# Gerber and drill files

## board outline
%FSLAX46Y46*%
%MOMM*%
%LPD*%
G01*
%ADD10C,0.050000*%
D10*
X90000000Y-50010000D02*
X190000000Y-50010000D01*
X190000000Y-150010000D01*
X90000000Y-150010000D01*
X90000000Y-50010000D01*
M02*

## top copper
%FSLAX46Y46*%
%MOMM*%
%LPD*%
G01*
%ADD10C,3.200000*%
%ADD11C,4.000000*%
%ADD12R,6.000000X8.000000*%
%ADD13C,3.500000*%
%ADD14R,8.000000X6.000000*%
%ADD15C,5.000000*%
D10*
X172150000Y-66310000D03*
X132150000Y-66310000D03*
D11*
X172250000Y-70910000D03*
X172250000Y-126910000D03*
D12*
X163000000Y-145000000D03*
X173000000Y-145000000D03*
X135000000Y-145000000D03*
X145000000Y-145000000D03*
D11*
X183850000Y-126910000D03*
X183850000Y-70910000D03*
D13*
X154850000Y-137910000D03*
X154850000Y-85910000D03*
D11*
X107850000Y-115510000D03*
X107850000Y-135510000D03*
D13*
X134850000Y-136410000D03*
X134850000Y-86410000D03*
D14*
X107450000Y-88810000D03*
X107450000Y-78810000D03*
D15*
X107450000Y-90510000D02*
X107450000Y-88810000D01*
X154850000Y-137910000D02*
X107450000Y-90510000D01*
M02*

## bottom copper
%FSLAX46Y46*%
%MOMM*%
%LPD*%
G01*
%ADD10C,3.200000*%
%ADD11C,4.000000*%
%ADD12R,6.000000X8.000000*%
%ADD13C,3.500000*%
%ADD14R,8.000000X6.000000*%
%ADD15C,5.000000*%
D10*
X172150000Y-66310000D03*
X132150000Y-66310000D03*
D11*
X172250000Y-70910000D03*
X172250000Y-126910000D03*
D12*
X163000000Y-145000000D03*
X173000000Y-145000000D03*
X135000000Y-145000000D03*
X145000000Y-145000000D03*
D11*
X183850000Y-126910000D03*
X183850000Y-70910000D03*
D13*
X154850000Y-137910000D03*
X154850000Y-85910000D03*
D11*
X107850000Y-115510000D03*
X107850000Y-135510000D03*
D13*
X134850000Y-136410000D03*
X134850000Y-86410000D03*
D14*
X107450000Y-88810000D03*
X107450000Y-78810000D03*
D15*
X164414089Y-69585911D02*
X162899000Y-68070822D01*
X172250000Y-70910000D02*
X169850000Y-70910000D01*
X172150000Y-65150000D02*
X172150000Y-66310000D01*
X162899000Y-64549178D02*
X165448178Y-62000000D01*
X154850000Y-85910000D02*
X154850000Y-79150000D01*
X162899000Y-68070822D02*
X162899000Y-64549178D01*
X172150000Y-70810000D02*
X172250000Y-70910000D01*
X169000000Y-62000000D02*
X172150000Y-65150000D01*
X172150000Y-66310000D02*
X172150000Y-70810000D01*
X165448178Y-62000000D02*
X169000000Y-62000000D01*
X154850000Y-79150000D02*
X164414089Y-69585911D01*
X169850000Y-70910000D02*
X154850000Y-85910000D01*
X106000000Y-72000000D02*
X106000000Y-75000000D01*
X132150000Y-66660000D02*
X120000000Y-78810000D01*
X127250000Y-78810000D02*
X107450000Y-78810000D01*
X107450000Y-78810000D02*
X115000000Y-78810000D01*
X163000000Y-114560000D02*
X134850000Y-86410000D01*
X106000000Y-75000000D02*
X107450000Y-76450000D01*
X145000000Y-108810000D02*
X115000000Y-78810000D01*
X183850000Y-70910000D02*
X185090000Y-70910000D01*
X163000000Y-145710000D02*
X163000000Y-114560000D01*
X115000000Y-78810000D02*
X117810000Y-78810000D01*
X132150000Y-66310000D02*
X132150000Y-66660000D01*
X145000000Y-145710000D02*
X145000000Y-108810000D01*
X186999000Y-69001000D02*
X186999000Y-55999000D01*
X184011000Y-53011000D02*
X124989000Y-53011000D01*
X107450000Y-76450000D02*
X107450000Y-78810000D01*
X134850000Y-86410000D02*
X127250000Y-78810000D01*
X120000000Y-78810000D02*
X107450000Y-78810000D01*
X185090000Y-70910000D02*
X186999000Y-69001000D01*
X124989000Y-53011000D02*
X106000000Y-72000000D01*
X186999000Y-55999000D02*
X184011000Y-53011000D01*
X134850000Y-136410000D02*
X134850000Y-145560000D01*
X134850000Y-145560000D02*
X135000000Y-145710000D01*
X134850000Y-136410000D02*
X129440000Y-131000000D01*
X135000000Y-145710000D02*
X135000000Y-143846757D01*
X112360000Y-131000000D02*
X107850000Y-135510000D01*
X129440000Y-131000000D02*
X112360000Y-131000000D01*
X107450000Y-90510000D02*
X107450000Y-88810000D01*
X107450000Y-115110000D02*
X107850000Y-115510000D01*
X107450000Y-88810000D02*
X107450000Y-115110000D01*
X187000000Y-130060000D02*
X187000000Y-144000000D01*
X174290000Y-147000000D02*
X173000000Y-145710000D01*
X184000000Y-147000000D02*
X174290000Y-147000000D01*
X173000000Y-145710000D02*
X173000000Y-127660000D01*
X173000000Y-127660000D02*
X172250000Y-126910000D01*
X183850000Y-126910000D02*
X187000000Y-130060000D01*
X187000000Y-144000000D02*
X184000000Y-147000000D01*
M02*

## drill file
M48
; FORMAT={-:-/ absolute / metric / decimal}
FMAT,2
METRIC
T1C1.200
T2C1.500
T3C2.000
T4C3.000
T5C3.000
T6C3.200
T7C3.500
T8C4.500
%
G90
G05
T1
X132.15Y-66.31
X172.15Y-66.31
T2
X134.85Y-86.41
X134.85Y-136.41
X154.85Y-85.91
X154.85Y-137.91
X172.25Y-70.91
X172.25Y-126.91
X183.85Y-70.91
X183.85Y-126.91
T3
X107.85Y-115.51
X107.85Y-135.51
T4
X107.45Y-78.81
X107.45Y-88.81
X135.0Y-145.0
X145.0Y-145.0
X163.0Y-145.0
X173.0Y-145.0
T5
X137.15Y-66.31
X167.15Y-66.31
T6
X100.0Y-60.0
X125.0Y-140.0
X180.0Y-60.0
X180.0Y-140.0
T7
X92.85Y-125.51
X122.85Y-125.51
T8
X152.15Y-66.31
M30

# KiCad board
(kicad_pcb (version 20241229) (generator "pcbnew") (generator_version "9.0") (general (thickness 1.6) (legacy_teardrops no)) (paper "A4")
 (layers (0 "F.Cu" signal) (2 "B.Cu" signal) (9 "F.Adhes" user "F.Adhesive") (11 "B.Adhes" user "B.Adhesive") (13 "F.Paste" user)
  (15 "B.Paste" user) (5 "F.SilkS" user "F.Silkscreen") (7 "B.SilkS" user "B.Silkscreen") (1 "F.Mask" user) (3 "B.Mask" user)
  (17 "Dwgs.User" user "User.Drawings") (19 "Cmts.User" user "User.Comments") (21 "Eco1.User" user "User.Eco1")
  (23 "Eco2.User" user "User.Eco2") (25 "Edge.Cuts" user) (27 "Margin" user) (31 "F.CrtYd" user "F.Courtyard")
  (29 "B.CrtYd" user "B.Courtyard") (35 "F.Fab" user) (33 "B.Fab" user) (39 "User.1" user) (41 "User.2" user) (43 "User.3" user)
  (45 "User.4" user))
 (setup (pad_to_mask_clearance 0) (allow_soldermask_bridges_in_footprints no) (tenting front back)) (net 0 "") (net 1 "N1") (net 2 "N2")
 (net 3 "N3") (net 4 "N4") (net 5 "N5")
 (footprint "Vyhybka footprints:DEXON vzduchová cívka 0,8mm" (layer "F.Cu") (at 152.15 66.31 180)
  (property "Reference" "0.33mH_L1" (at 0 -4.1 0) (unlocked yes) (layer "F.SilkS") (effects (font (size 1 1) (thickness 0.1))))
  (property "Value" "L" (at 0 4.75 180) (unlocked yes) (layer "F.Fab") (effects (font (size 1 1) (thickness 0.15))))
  (pad "" np_thru_hole circle (at -15 0 180) (size 3 3) (drill 3) (layers "*.Cu" "*.Mask"))
  (pad "" np_thru_hole circle (at 0 0 180) (size 4.5 4.5) (drill 4.5) (layers "*.Cu" "*.Mask"))
  (pad "" np_thru_hole circle (at 15 0 180) (size 3 3) (drill 3) (layers "*.Cu" "*.Mask"))
  (pad "1" thru_hole circle (at -20 0 180) (size 3.2 3.2) (drill 1.2) (layers "*.Cu" "*.Mask") (remove_unused_layers no) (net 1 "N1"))
  (pad "2" thru_hole circle (at 20 0 180) (size 3.2 3.2) (drill 1.2) (layers "*.Cu" "*.Mask") (remove_unused_layers no) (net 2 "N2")))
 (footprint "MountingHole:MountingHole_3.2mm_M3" (layer "F.Cu") (at 180 60)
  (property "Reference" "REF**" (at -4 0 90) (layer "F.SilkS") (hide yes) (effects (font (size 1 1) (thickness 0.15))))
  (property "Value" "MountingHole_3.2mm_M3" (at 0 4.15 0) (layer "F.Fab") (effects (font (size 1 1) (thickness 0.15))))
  (pad "" np_thru_hole circle (at 0 0) (size 3.2 3.2) (drill 3.2) (layers "*.Cu" "*.Mask")))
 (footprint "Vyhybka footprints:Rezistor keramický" (layer "F.Cu") (at 172.25 98.91 -90)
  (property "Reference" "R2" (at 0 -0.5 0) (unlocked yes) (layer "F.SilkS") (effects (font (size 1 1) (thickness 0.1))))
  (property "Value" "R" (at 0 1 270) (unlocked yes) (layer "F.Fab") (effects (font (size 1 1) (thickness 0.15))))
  (pad "1" thru_hole circle (at -28 0 270) (size 4 4) (drill 1.5) (layers "*.Cu" "*.Mask") (remove_unused_layers no) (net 1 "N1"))
  (pad "2" thru_hole circle (at 28 0 270) (size 4 4) (drill 1.5) (layers "*.Cu" "*.Mask") (remove_unused_layers no) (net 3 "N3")))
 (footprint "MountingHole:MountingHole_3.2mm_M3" (layer "F.Cu") (at 100 60)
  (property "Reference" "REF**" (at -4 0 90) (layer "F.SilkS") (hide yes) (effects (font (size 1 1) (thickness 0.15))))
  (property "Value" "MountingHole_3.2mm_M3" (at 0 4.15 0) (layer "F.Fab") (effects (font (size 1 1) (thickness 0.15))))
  (pad "" np_thru_hole circle (at 0 0) (size 3.2 3.2) (drill 3.2) (layers "*.Cu" "*.Mask")))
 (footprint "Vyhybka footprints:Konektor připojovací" (layer "F.Cu") (at 168 145)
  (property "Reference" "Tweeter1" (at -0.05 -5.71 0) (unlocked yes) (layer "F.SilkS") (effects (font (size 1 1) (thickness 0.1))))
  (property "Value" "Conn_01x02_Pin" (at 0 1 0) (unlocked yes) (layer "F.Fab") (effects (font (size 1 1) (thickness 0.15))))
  (pad "1" thru_hole rect (at -5 0) (size 6 8) (drill 3) (layers "*.Cu" "*.Mask") (remove_unused_layers no) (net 2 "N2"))
  (pad "2" thru_hole rect (at 5 0) (size 6 8) (drill 3) (layers "*.Cu" "*.Mask") (remove_unused_layers no) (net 3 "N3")))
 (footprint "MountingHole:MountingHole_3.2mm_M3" (layer "F.Cu") (at 125 140)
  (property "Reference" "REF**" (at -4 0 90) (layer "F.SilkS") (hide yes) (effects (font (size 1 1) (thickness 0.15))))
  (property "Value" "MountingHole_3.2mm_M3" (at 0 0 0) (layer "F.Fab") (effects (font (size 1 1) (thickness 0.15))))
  (pad "" np_thru_hole circle (at 0 0) (size 3.2 3.2) (drill 3.2) (layers "*.Cu" "*.Mask")))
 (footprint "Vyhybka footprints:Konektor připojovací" (layer "F.Cu") (at 140 145)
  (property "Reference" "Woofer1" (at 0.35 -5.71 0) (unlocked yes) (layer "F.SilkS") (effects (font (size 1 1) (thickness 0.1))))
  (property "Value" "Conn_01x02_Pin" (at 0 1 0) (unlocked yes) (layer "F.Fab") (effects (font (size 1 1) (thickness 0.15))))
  (pad "1" thru_hole rect (at -5 0) (size 6 8) (drill 3) (layers "*.Cu" "*.Mask") (remove_unused_layers no) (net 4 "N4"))
  (pad "2" thru_hole rect (at 5 0) (size 6 8) (drill 3) (layers "*.Cu" "*.Mask") (remove_unused_layers no) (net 2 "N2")))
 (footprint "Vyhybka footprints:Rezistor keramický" (layer "F.Cu") (at 183.85 98.91 90)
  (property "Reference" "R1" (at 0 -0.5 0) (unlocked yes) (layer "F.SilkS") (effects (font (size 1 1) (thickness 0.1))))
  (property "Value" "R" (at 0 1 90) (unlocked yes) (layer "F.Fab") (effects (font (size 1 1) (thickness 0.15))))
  (pad "1" thru_hole circle (at -28 0 90) (size 4 4) (drill 1.5) (layers "*.Cu" "*.Mask") (remove_unused_layers no) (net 3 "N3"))
  (pad "2" thru_hole circle (at 28 0 90) (size 4 4) (drill 1.5) (layers "*.Cu" "*.Mask") (remove_unused_layers no) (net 2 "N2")))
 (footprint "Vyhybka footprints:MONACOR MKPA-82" (layer "F.Cu") (at 154.85 111.91 90)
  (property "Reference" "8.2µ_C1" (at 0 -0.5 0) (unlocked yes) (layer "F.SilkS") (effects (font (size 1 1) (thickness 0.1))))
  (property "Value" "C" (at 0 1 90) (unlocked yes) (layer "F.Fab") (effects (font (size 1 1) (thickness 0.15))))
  (pad "1" thru_hole circle (at -26 0 90) (size 3.5 3.5) (drill 1.5) (layers "*.Cu" "*.Mask") (remove_unused_layers no) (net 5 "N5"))
  (pad "2" thru_hole circle (at 26 0 90) (size 3.5 3.5) (drill 1.5) (layers "*.Cu" "*.Mask") (remove_unused_layers no) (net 1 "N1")))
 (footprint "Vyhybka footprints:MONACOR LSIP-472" (layer "F.Cu") (at 107.85 125.51 -90)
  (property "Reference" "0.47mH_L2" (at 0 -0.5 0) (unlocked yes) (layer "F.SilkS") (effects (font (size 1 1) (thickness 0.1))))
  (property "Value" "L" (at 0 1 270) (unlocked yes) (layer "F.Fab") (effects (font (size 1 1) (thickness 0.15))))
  (pad "" np_thru_hole circle (at 0 -15 270) (size 3.5 3.5) (drill 3.5) (layers "*.Cu" "*.Mask"))
  (pad "" np_thru_hole circle (at 0 15 270) (size 3.5 3.5) (drill 3.5) (layers "*.Cu" "*.Mask"))
  (pad "1" thru_hole circle (at -10 0 270) (size 4 4) (drill 2) (layers "*.Cu" "*.Mask") (remove_unused_layers no) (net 5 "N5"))
  (pad "2" thru_hole circle (at 10 0 270) (size 4 4) (drill 2) (layers "*.Cu" "*.Mask") (remove_unused_layers no) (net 4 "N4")))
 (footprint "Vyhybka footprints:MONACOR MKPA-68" (layer "F.Cu") (at 134.85 111.41 90)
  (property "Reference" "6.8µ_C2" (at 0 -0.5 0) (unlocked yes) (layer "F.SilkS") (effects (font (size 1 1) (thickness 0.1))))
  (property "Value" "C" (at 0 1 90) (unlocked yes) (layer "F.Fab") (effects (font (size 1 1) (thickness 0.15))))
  (pad "1" thru_hole circle (at -25 0 90) (size 3.5 3.5) (drill 1.5) (layers "*.Cu" "*.Mask") (remove_unused_layers no) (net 4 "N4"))
  (pad "2" thru_hole circle (at 25 0 90) (size 3.5 3.5) (drill 1.5) (layers "*.Cu" "*.Mask") (remove_unused_layers no) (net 2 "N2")))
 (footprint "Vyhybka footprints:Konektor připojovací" (layer "F.Cu") (at 107.45 83.81 90)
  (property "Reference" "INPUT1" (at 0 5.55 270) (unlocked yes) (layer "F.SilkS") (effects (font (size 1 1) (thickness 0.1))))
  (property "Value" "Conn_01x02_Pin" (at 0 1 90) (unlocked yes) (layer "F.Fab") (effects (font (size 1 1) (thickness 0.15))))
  (pad "1" thru_hole rect (at -5 0 90) (size 6 8) (drill 3) (layers "*.Cu" "*.Mask") (remove_unused_layers no) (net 5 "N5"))
  (pad "2" thru_hole rect (at 5 0 90) (size 6 8) (drill 3) (layers "*.Cu" "*.Mask") (remove_unused_layers no) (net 2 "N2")))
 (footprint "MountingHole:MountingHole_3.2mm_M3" (layer "F.Cu") (at 180 140)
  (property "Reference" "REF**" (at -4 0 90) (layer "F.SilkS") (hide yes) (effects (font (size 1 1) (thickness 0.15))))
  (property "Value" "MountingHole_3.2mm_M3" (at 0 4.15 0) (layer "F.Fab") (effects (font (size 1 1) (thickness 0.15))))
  (pad "" np_thru_hole circle (at 0 0) (size 3.2 3.2) (drill 3.2) (layers "*.Cu" "*.Mask")))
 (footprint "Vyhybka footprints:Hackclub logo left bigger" (layer "F.Cu") (at 102 69)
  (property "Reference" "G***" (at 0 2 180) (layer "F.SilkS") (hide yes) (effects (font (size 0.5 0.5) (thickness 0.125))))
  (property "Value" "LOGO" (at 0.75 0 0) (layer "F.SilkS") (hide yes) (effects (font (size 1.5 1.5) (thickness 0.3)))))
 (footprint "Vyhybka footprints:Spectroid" (layer "B.Cu") (at 98 137 180)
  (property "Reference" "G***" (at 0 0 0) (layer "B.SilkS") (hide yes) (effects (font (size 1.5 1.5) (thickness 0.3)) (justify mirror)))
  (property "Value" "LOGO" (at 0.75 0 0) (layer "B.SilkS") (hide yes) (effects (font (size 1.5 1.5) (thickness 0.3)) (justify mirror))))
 (gr_rect (start 90 50.01) (end 190 150.01) (stroke (width 0.05) (type default)) (fill no) (layer "Edge.Cuts"))
 (segment (start 164.414089 69.585911) (end 162.899 68.070822) (width 5) (layer "B.Cu") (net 1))
 (segment (start 172.25 70.91) (end 169.85 70.91) (width 5) (layer "B.Cu") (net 1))
 (segment (start 172.15 65.15) (end 172.15 66.31) (width 5) (layer "B.Cu") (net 1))
 (segment (start 162.899 64.549178) (end 165.448178 62) (width 5) (layer "B.Cu") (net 1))
 (segment (start 154.85 85.91) (end 154.85 79.15) (width 5) (layer "B.Cu") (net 1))
 (segment (start 162.899 68.070822) (end 162.899 64.549178) (width 5) (layer "B.Cu") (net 1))
 (segment (start 172.15 70.81) (end 172.25 70.91) (width 5) (layer "B.Cu") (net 1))
 (segment (start 169 62) (end 172.15 65.15) (width 5) (layer "B.Cu") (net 1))
 (segment (start 172.15 66.31) (end 172.15 70.81) (width 5) (layer "B.Cu") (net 1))
 (segment (start 165.448178 62) (end 169 62) (width 5) (layer "B.Cu") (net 1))
 (segment (start 154.85 79.15) (end 164.414089 69.585911) (width 5) (layer "B.Cu") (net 1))
 (segment (start 169.85 70.91) (end 154.85 85.91) (width 5) (layer "B.Cu") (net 1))
 (segment (start 106 72) (end 106 75) (width 5) (layer "B.Cu") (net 2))
 (segment (start 132.15 66.66) (end 120 78.81) (width 5) (layer "B.Cu") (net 2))
 (segment (start 127.25 78.81) (end 107.45 78.81) (width 5) (layer "B.Cu") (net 2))
 (segment (start 107.45 78.81) (end 115 78.81) (width 5) (layer "B.Cu") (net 2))
 (segment (start 163 114.56) (end 134.85 86.41) (width 5) (layer "B.Cu") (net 2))
 (segment (start 106 75) (end 107.45 76.45) (width 5) (layer "B.Cu") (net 2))
 (segment (start 145 108.81) (end 115 78.81) (width 5) (layer "B.Cu") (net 2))
 (segment (start 183.85 70.91) (end 185.09 70.91) (width 5) (layer "B.Cu") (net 2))
 (segment (start 163 145.71) (end 163 114.56) (width 5) (layer "B.Cu") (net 2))
 (segment (start 115 78.81) (end 117.81 78.81) (width 5) (layer "B.Cu") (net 2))
 (segment (start 132.15 66.31) (end 132.15 66.66) (width 5) (layer "B.Cu") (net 2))
 (segment (start 145 145.71) (end 145 108.81) (width 5) (layer "B.Cu") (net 2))
 (segment (start 186.999 69.001) (end 186.999 55.999) (width 5) (layer "B.Cu") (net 2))
 (segment (start 184.011 53.011) (end 124.989 53.011) (width 5) (layer "B.Cu") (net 2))
 (segment (start 107.45 76.45) (end 107.45 78.81) (width 5) (layer "B.Cu") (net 2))
 (segment (start 134.85 86.41) (end 127.25 78.81) (width 5) (layer "B.Cu") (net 2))
 (segment (start 120 78.81) (end 107.45 78.81) (width 5) (layer "B.Cu") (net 2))
 (segment (start 185.09 70.91) (end 186.999 69.001) (width 5) (layer "B.Cu") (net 2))
 (segment (start 124.989 53.011) (end 106 72) (width 5) (layer "B.Cu") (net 2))
 (segment (start 186.999 55.999) (end 184.011 53.011) (width 5) (layer "B.Cu") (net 2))
 (segment (start 134.85 136.41) (end 134.85 145.56) (width 5) (layer "B.Cu") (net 4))
 (segment (start 134.85 145.56) (end 135 145.71) (width 5) (layer "B.Cu") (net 4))
 (segment (start 134.85 136.41) (end 129.44 131) (width 5) (layer "B.Cu") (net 4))
 (segment (start 135 145.71) (end 135 143.846757) (width 5) (layer "B.Cu") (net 4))
 (segment (start 112.36 131) (end 107.85 135.51) (width 5) (layer "B.Cu") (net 4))
 (segment (start 129.44 131) (end 112.36 131) (width 5) (layer "B.Cu") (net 4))
 (segment (start 107.45 90.51) (end 107.45 88.81) (width 5) (layer "F.Cu") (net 5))
 (segment (start 154.85 137.91) (end 107.45 90.51) (width 5) (layer "F.Cu") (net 5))
 (segment (start 107.45 90.51) (end 107.45 88.81) (width 5) (layer "B.Cu") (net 5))
 (segment (start 107.45 115.11) (end 107.85 115.51) (width 5) (layer "B.Cu") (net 5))
 (segment (start 107.45 88.81) (end 107.45 115.11) (width 5) (layer "B.Cu") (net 5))
 (segment (start 187 130.06) (end 187 144) (width 5) (layer "B.Cu") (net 3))
 (segment (start 174.29 147) (end 173 145.71) (width 5) (layer "B.Cu") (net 3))
 (segment (start 184 147) (end 174.29 147) (width 5) (layer "B.Cu") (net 3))
 (segment (start 173 145.71) (end 173 127.66) (width 5) (layer "B.Cu") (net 3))
 (segment (start 173 127.66) (end 172.25 126.91) (width 5) (layer "B.Cu") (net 3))
 (segment (start 183.85 126.91) (end 187 130.06) (width 5) (layer "B.Cu") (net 3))
 (segment (start 187 144) (end 184 147) (width 5) (layer "B.Cu") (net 3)))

